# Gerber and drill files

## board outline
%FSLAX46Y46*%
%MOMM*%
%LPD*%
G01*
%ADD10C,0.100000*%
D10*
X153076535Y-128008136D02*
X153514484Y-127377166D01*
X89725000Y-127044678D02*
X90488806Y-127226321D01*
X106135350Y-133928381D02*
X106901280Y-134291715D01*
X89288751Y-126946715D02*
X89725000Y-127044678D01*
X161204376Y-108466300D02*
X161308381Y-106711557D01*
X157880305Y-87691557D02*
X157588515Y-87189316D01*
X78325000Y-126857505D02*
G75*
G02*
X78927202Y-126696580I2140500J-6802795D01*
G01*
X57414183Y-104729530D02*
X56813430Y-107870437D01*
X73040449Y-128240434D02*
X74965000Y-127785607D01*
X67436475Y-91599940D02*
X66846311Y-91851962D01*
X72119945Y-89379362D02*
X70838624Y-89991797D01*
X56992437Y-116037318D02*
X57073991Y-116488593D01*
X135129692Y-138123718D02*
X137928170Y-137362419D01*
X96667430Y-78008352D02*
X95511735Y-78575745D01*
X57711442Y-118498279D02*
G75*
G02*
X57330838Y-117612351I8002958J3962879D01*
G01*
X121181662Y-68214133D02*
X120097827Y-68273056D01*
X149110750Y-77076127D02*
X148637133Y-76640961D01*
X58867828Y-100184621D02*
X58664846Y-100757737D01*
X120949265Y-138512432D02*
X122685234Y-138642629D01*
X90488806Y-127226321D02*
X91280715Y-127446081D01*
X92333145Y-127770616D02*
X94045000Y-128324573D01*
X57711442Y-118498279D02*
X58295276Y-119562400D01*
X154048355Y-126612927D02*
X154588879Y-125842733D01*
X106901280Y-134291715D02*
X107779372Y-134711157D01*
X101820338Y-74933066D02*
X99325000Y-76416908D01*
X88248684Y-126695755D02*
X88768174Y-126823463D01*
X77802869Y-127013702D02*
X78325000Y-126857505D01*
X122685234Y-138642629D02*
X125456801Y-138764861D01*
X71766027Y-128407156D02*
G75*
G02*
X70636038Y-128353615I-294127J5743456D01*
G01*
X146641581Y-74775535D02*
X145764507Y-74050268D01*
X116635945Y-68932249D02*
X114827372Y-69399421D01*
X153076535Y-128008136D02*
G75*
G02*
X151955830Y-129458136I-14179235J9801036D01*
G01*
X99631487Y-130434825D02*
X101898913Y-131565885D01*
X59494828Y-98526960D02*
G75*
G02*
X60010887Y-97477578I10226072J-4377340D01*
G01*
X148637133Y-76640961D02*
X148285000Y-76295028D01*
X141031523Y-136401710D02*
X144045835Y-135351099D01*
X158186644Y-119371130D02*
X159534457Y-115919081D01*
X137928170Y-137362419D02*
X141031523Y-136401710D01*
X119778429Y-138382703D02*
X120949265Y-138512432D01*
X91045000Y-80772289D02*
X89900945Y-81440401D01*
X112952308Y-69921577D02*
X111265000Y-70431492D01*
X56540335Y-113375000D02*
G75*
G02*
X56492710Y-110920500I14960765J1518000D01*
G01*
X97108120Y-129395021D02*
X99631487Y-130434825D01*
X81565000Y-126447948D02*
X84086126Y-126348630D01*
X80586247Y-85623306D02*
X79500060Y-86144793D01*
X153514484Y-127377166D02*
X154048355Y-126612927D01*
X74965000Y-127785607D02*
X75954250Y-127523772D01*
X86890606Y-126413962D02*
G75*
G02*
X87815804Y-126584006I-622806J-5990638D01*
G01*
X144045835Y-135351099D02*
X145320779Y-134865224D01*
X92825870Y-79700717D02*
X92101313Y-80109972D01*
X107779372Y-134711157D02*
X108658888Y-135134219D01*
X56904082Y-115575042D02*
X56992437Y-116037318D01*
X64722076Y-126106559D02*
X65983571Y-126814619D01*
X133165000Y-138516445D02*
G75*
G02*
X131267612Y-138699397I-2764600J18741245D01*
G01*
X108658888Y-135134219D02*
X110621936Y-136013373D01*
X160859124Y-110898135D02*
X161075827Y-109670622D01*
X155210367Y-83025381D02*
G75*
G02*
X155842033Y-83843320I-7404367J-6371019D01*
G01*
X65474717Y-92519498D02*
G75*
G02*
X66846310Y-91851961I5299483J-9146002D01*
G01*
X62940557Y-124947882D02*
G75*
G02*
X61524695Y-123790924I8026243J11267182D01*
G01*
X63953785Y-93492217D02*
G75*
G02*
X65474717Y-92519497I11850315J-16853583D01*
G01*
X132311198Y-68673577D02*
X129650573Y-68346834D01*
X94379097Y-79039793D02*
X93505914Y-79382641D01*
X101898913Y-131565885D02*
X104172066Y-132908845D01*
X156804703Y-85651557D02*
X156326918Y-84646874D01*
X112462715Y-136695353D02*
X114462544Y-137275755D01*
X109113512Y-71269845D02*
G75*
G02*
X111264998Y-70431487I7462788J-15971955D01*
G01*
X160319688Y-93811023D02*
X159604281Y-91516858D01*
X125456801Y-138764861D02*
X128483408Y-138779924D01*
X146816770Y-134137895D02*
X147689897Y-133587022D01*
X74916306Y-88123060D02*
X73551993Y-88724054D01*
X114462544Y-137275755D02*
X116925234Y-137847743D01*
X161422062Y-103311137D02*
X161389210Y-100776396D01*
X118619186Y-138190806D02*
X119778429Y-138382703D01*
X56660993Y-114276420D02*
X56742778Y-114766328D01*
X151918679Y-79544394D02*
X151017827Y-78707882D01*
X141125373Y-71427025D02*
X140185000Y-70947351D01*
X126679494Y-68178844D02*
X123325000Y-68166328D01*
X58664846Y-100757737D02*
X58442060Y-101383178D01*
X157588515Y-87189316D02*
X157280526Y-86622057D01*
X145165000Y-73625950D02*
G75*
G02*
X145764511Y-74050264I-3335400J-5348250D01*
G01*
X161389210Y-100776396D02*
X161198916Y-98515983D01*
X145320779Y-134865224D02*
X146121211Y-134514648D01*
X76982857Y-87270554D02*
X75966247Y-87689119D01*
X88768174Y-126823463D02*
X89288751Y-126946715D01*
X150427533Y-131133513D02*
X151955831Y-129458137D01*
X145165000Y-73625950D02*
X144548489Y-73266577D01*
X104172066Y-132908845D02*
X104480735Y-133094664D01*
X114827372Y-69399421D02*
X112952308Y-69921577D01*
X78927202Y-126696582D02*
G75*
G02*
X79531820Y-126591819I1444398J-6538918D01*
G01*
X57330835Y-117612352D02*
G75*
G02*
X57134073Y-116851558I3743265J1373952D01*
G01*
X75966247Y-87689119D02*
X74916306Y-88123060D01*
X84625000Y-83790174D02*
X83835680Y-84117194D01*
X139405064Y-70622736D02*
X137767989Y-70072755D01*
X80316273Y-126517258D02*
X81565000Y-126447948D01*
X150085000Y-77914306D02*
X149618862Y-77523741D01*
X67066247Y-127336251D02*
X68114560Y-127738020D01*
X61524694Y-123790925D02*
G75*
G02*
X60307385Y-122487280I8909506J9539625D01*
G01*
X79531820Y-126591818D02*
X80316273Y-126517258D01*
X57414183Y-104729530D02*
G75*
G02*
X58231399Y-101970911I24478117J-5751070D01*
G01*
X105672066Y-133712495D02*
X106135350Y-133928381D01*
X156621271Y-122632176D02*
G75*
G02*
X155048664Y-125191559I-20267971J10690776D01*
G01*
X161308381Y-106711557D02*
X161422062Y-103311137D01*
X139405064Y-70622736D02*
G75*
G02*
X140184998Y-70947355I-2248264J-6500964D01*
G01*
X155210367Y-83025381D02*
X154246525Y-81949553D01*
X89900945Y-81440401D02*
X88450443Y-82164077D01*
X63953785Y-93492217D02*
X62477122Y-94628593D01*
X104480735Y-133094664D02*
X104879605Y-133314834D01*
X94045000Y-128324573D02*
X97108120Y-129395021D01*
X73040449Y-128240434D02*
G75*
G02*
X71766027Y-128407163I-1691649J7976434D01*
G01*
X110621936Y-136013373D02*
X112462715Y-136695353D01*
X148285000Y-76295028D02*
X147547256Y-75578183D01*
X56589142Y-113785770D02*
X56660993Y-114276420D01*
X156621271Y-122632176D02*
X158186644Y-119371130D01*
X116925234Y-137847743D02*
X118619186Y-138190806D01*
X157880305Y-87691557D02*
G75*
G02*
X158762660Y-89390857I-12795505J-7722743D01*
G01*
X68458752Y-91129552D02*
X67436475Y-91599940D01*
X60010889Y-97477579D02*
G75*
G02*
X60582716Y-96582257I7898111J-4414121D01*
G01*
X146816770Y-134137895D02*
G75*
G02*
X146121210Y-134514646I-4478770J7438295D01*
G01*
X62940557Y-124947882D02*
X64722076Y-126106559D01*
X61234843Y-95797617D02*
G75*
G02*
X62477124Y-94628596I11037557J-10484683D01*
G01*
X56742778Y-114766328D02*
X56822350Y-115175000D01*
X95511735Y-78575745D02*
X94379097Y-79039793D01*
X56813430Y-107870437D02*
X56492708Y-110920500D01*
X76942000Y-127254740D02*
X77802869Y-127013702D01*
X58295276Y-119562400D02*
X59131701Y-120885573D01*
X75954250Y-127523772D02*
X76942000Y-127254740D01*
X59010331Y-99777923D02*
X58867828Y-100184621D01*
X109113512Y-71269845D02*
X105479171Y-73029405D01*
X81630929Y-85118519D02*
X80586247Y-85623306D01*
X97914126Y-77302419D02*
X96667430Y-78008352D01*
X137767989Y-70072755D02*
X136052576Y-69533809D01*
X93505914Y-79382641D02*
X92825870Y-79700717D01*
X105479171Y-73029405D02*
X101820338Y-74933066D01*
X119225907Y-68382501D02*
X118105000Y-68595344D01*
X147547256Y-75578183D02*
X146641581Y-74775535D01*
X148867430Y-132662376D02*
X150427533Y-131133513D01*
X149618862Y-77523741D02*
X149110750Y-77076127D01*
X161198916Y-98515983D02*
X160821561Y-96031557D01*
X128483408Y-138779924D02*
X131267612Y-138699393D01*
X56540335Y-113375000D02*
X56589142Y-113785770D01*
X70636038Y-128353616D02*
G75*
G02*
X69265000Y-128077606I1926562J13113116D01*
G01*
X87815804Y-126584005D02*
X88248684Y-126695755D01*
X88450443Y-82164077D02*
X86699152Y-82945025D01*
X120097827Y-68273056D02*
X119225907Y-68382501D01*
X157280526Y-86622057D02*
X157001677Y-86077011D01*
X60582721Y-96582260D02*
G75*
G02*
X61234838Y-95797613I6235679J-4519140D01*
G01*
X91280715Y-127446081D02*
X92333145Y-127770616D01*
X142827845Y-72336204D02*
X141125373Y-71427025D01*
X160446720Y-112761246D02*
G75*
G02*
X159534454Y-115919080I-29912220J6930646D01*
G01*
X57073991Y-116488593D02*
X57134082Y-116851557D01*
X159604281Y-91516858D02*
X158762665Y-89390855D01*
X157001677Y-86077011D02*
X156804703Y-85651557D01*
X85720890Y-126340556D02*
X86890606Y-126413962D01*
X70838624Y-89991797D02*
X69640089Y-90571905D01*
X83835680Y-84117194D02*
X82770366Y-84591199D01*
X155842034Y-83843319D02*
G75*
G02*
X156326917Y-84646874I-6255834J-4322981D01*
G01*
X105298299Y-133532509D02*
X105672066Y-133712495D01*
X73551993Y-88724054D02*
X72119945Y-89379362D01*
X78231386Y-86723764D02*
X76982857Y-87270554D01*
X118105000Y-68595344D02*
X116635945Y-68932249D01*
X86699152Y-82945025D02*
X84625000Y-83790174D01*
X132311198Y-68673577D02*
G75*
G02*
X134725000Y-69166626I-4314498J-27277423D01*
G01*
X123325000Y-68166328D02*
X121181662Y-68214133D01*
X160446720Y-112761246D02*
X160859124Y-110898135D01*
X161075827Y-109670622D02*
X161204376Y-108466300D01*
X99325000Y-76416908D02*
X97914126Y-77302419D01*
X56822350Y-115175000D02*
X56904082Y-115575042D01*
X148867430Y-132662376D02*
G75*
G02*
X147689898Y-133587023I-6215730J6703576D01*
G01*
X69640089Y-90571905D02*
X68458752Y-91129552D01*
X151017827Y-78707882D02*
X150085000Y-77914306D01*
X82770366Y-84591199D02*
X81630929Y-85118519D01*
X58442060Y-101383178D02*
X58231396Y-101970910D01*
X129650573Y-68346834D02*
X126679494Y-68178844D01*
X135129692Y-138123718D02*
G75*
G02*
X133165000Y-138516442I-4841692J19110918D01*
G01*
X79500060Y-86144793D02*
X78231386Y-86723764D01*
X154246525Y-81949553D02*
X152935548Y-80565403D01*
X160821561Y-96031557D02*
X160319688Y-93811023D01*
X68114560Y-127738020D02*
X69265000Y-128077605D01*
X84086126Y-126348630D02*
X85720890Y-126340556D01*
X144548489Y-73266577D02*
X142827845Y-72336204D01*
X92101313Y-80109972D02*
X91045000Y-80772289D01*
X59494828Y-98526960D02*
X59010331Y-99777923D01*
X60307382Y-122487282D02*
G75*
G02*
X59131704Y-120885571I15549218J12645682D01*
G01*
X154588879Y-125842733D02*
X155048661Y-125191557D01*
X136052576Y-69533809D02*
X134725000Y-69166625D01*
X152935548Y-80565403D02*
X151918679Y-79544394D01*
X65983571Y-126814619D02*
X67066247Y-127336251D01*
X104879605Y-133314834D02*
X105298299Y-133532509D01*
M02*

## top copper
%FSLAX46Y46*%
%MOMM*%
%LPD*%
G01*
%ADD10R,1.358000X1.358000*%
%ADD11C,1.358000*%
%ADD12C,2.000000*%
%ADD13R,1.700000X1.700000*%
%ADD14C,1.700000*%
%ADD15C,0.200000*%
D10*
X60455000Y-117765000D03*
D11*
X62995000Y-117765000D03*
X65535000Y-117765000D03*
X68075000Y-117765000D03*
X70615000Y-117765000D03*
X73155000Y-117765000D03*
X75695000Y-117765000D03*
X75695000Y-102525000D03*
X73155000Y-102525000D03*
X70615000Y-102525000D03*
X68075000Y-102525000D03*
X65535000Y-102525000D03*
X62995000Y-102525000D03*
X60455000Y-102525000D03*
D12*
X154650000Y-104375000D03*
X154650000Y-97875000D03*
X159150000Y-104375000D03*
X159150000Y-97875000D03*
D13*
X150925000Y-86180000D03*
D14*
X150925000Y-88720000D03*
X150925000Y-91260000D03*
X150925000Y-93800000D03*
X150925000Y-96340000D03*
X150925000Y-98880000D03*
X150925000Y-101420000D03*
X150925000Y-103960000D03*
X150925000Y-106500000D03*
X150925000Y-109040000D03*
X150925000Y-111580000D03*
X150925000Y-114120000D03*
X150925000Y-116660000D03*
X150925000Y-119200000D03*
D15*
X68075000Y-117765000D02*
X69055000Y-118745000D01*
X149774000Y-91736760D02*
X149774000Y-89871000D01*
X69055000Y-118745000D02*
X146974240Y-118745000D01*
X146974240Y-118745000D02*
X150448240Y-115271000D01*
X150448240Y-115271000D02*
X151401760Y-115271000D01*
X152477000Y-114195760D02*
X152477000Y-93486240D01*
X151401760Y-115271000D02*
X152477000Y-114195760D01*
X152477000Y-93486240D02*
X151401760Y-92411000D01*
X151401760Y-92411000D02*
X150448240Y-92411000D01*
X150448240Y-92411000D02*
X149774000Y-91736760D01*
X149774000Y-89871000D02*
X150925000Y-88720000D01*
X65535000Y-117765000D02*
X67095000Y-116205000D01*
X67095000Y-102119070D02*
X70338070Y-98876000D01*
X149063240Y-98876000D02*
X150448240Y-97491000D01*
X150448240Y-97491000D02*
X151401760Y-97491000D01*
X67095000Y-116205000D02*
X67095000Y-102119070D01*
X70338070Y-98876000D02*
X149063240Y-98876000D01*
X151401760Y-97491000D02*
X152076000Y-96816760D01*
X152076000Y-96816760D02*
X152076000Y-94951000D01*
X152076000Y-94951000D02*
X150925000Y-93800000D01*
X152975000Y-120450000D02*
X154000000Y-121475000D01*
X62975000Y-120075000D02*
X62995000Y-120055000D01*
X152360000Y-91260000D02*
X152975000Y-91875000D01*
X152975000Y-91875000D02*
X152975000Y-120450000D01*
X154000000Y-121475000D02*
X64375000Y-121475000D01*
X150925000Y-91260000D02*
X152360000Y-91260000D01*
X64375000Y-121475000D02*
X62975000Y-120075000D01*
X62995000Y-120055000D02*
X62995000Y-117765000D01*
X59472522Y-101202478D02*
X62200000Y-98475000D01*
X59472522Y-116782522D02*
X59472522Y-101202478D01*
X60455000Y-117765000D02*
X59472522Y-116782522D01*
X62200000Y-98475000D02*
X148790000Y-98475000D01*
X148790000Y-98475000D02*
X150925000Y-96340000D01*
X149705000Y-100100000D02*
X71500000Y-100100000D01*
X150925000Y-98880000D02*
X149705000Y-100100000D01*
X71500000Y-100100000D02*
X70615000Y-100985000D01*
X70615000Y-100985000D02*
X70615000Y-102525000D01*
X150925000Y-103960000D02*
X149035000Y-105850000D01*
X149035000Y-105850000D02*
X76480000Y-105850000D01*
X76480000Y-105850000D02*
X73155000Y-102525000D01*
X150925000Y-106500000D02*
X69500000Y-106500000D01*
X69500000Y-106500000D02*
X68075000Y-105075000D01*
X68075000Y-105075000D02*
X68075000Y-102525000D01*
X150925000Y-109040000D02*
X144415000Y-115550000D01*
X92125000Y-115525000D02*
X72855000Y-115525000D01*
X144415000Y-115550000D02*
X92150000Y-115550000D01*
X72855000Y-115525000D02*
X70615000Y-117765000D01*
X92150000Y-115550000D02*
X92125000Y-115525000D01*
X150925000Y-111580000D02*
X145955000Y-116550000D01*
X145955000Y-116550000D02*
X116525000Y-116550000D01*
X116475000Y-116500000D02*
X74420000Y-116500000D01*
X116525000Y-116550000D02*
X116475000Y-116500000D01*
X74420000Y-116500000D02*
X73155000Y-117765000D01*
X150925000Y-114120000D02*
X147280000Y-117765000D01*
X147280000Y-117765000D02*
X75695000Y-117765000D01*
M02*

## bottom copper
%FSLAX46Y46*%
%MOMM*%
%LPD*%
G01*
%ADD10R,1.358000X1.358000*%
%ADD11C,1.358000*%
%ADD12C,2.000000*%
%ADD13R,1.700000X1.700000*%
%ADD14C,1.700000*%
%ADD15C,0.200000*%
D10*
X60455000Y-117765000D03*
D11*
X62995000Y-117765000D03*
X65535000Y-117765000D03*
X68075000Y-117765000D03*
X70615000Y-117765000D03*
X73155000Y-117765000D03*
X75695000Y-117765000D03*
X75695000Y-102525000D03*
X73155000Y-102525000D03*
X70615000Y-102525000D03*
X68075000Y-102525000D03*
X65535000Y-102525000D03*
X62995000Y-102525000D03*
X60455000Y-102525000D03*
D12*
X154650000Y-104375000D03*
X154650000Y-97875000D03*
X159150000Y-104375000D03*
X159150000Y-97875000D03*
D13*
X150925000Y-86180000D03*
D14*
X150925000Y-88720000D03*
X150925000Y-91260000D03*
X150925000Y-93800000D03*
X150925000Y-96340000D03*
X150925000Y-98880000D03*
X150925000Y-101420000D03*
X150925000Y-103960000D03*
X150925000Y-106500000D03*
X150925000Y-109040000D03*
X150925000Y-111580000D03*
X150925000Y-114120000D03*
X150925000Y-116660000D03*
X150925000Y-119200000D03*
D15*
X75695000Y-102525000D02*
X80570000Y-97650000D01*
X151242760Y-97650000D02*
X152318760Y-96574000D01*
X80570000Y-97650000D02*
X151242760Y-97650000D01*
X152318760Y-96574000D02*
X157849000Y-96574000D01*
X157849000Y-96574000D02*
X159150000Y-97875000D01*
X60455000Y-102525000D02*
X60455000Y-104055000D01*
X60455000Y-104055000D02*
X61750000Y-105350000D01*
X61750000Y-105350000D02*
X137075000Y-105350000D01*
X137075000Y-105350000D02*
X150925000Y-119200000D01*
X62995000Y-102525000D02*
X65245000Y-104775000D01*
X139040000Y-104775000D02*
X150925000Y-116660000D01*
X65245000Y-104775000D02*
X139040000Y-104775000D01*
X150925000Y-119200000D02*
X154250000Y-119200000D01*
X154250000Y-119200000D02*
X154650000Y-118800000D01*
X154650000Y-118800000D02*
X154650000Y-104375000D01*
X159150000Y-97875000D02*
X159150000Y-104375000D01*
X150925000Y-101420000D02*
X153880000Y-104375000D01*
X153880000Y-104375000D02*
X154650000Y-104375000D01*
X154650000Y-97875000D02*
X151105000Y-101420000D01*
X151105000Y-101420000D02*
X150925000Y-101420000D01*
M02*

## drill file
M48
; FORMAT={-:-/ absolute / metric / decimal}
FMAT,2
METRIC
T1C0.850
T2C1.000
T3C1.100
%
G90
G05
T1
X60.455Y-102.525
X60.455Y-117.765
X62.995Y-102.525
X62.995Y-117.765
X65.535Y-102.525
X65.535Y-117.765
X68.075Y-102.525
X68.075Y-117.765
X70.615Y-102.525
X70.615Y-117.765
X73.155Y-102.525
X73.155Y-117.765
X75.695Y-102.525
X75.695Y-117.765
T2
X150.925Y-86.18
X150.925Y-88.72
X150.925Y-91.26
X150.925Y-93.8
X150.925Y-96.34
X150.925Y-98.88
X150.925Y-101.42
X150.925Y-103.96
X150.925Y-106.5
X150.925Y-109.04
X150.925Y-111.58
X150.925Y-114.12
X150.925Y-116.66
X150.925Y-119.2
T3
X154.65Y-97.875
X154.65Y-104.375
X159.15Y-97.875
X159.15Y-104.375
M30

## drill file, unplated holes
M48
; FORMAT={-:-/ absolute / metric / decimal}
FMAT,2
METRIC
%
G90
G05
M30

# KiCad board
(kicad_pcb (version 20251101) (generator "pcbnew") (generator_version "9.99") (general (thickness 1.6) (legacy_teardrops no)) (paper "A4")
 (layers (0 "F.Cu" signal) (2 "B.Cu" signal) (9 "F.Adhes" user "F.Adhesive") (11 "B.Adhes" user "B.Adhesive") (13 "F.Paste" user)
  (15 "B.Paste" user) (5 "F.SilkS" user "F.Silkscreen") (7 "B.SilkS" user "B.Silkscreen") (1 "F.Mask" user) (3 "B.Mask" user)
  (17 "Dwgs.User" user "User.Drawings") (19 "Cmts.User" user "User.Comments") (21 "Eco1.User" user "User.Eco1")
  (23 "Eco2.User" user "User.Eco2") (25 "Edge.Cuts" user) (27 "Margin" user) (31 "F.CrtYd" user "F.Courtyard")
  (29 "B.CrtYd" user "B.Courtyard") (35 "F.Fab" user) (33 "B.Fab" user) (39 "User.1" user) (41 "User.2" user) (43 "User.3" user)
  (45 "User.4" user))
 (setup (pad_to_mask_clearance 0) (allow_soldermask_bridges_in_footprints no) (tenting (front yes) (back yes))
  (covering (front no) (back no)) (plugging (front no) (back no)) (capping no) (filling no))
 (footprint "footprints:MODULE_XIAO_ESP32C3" (layer "F.Cu") (at 68.0115 110.145 90)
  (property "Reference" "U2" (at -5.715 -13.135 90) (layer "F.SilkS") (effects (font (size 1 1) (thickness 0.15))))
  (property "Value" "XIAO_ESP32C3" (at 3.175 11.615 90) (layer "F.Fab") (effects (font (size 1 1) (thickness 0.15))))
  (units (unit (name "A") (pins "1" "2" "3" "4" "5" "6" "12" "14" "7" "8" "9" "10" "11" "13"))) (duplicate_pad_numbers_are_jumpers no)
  (pad "1" thru_hole rect (at -7.62 -7.5565 90) (size 1.358 1.358) (drill 0.85) (layers "*.Cu" "*.Mask") (remove_unused_layers no)
   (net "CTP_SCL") (solder_mask_margin 0.102) (tenting (front none) (back none)))
  (pad "2" thru_hole circle (at -7.62 -5.0165 90) (size 1.358 1.358) (drill 0.85) (layers "*.Cu" "*.Mask") (remove_unused_layers no)
   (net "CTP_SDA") (solder_mask_margin 0.102) (tenting (front none) (back none)))
  (pad "3" thru_hole circle (at -7.62 -2.4765 90) (size 1.358 1.358) (drill 0.85) (layers "*.Cu" "*.Mask") (remove_unused_layers no)
   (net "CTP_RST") (solder_mask_margin 0.102) (tenting (front none) (back none)))
  (pad "4" thru_hole circle (at -7.62 0.0635 90) (size 1.358 1.358) (drill 0.85) (layers "*.Cu" "*.Mask") (remove_unused_layers no)
   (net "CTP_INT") (solder_mask_margin 0.102) (tenting (front none) (back none)))
  (pad "5" thru_hole circle (at -7.62 2.6035 90) (size 1.358 1.358) (drill 0.85) (layers "*.Cu" "*.Mask") (remove_unused_layers no)
   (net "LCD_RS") (solder_mask_margin 0.102) (tenting (front none) (back none)))
  (pad "6" thru_hole circle (at -7.62 5.1435 90) (size 1.358 1.358) (drill 0.85) (layers "*.Cu" "*.Mask") (remove_unused_layers no)
   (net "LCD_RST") (solder_mask_margin 0.102) (tenting (front none) (back none)))
  (pad "7" thru_hole circle (at -7.62 7.6835 90) (size 1.358 1.358) (drill 0.85) (layers "*.Cu" "*.Mask") (remove_unused_layers no)
   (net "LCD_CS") (solder_mask_margin 0.102) (tenting (front none) (back none)))
  (pad "8" thru_hole circle (at 7.62 7.6835 90) (size 1.358 1.358) (drill 0.85) (layers "*.Cu" "*.Mask") (remove_unused_layers no)
   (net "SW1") (solder_mask_margin 0.102) (tenting (front none) (back none)))
  (pad "9" thru_hole circle (at 7.62 5.1435 90) (size 1.358 1.358) (drill 0.85) (layers "*.Cu" "*.Mask") (remove_unused_layers no)
   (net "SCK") (solder_mask_margin 0.102) (tenting (front none) (back none)))
  (pad "10" thru_hole circle (at 7.62 2.6035 90) (size 1.358 1.358) (drill 0.85) (layers "*.Cu" "*.Mask") (remove_unused_layers no)
   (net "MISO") (solder_mask_margin 0.102) (tenting (front none) (back none)))
  (pad "11" thru_hole circle (at 7.62 0.0635 90) (size 1.358 1.358) (drill 0.85) (layers "*.Cu" "*.Mask") (remove_unused_layers no)
   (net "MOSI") (solder_mask_margin 0.102) (tenting (front none) (back none)))
  (pad "12" thru_hole circle (at 7.62 -2.4765 90) (size 1.358 1.358) (drill 0.85) (layers "*.Cu" "*.Mask") (remove_unused_layers no)
   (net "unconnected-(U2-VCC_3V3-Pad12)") (solder_mask_margin 0.102) (tenting (front none) (back none)))
  (pad "13" thru_hole circle (at 7.62 -5.0165 90) (size 1.358 1.358) (drill 0.85) (layers "*.Cu" "*.Mask") (remove_unused_layers no)
   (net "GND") (solder_mask_margin 0.102) (tenting (front none) (back none)))
  (pad "14" thru_hole circle (at 7.62 -7.5565 90) (size 1.358 1.358) (drill 0.85) (layers "*.Cu" "*.Mask") (remove_unused_layers no)
   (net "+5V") (solder_mask_margin 0.102) (tenting (front none) (back none))))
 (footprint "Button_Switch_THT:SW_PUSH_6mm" (layer "F.Cu") (at 154.65 104.375 90)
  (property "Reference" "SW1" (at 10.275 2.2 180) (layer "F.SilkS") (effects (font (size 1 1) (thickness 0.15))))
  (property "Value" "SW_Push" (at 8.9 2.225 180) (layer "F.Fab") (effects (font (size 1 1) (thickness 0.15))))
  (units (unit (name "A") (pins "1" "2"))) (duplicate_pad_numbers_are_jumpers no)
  (pad "1" thru_hole circle (at 0 0 180) (size 2 2) (drill 1.1) (layers "*.Cu" "*.Mask") (remove_unused_layers no) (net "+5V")
   (tenting (front none) (back none)))
  (pad "1" thru_hole circle (at 6.5 0 180) (size 2 2) (drill 1.1) (layers "*.Cu" "*.Mask") (remove_unused_layers no) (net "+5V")
   (tenting (front none) (back none)))
  (pad "2" thru_hole circle (at 0 4.5 180) (size 2 2) (drill 1.1) (layers "*.Cu" "*.Mask") (remove_unused_layers no) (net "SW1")
   (tenting (front none) (back none)))
  (pad "2" thru_hole circle (at 6.5 4.5 180) (size 2 2) (drill 1.1) (layers "*.Cu" "*.Mask") (remove_unused_layers no) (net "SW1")
   (tenting (front none) (back none))))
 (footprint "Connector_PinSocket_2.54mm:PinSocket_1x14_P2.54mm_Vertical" (layer "F.Cu") (at 150.925 86.18)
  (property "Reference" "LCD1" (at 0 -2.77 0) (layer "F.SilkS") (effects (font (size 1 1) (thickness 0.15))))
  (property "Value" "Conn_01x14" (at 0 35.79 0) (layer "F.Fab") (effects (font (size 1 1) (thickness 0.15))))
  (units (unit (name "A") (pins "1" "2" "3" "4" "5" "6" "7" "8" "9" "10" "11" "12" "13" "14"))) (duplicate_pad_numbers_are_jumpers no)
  (pad "1" thru_hole rect (at 0 0) (size 1.7 1.7) (drill 1) (layers "*.Cu" "*.Mask") (remove_unused_layers no)
   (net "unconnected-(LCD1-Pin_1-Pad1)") (tenting (front none) (back none)))
  (pad "2" thru_hole circle (at 0 2.54) (size 1.7 1.7) (drill 1) (layers "*.Cu" "*.Mask") (remove_unused_layers no) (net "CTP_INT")
   (tenting (front none) (back none)))
  (pad "3" thru_hole circle (at 0 5.08) (size 1.7 1.7) (drill 1) (layers "*.Cu" "*.Mask") (remove_unused_layers no) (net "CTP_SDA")
   (tenting (front none) (back none)))
  (pad "4" thru_hole circle (at 0 7.62) (size 1.7 1.7) (drill 1) (layers "*.Cu" "*.Mask") (remove_unused_layers no) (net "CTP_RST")
   (tenting (front none) (back none)))
  (pad "5" thru_hole circle (at 0 10.16) (size 1.7 1.7) (drill 1) (layers "*.Cu" "*.Mask") (remove_unused_layers no) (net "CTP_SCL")
   (tenting (front none) (back none)))
  (pad "6" thru_hole circle (at 0 12.7) (size 1.7 1.7) (drill 1) (layers "*.Cu" "*.Mask") (remove_unused_layers no) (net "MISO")
   (tenting (front none) (back none)))
  (pad "7" thru_hole circle (at 0 15.24) (size 1.7 1.7) (drill 1) (layers "*.Cu" "*.Mask") (remove_unused_layers no) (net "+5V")
   (tenting (front none) (back none)))
  (pad "8" thru_hole circle (at 0 17.78) (size 1.7 1.7) (drill 1) (layers "*.Cu" "*.Mask") (remove_unused_layers no) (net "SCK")
   (tenting (front none) (back none)))
  (pad "9" thru_hole circle (at 0 20.32) (size 1.7 1.7) (drill 1) (layers "*.Cu" "*.Mask") (remove_unused_layers no) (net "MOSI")
   (tenting (front none) (back none)))
  (pad "10" thru_hole circle (at 0 22.86) (size 1.7 1.7) (drill 1) (layers "*.Cu" "*.Mask") (remove_unused_layers no) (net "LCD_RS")
   (tenting (front none) (back none)))
  (pad "11" thru_hole circle (at 0 25.4) (size 1.7 1.7) (drill 1) (layers "*.Cu" "*.Mask") (remove_unused_layers no) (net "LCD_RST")
   (tenting (front none) (back none)))
  (pad "12" thru_hole circle (at 0 27.94) (size 1.7 1.7) (drill 1) (layers "*.Cu" "*.Mask") (remove_unused_layers no) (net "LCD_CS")
   (tenting (front none) (back none)))
  (pad "13" thru_hole circle (at 0 30.48) (size 1.7 1.7) (drill 1) (layers "*.Cu" "*.Mask") (remove_unused_layers no) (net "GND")
   (tenting (front none) (back none)))
  (pad "14" thru_hole circle (at 0 33.02) (size 1.7 1.7) (drill 1) (layers "*.Cu" "*.Mask") (remove_unused_layers no) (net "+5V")
   (tenting (front none) (back none))))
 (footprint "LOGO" (layer "B.Cu") (at 118.27759 103.45 -90)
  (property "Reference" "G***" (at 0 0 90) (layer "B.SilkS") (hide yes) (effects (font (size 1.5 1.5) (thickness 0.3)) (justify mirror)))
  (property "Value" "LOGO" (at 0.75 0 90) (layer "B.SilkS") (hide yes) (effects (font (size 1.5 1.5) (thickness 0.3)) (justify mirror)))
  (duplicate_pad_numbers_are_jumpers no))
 (gr_line (start 153.076535 128.008136) (end 153.514484 127.377166) (stroke (width 0.1) (type default)) (layer "Edge.Cuts"))
 (gr_line (start 89.725 127.044678) (end 90.488806 127.226321) (stroke (width 0.1) (type default)) (layer "Edge.Cuts"))
 (gr_line (start 106.13535 133.928381) (end 106.90128 134.291715) (stroke (width 0.1) (type default)) (layer "Edge.Cuts"))
 (gr_line (start 89.288751 126.946715) (end 89.725 127.044678) (stroke (width 0.1) (type default)) (layer "Edge.Cuts"))
 (gr_line (start 161.204376 108.4663) (end 161.308381 106.711557) (stroke (width 0.1) (type default)) (layer "Edge.Cuts"))
 (gr_line (start 157.880305 87.691557) (end 157.588515 87.189316) (stroke (width 0.1) (type default)) (layer "Edge.Cuts"))
 (gr_arc (start 78.325 126.857505) (mid 78.624342 126.770461) (end 78.927202 126.696582) (stroke (width 0.1) (type default))
  (layer "Edge.Cuts"))
 (gr_line (start 57.414183 104.72953) (end 56.81343 107.870437) (stroke (width 0.1) (type default)) (layer "Edge.Cuts"))
 (gr_line (start 73.040449 128.240434) (end 74.965 127.785607) (stroke (width 0.1) (type default)) (layer "Edge.Cuts"))
 (gr_line (start 67.436475 91.59994) (end 66.846311 91.851962) (stroke (width 0.1) (type default)) (layer "Edge.Cuts"))
 (gr_line (start 72.119945 89.379362) (end 70.838624 89.991797) (stroke (width 0.1) (type default)) (layer "Edge.Cuts"))
 (gr_line (start 56.992437 116.037318) (end 57.073991 116.488593) (stroke (width 0.1) (type default)) (layer "Edge.Cuts"))
 (gr_line (start 135.129692 138.123718) (end 137.92817 137.362419) (stroke (width 0.1) (type default)) (layer "Edge.Cuts"))
 (gr_line (start 96.66743 78.008352) (end 95.511735 78.575745) (stroke (width 0.1) (type default)) (layer "Edge.Cuts"))
 (gr_arc (start 57.711442 118.498279) (mid 57.509173 118.060456) (end 57.330835 117.612352) (stroke (width 0.1) (type default))
  (layer "Edge.Cuts"))
 (gr_line (start 121.181662 68.214133) (end 120.097827 68.273056) (stroke (width 0.1) (type default)) (layer "Edge.Cuts"))
 (gr_line (start 149.11075 77.076127) (end 148.637133 76.640961) (stroke (width 0.1) (type default)) (layer "Edge.Cuts"))
 (gr_line (start 58.867828 100.184621) (end 58.664846 100.757737) (stroke (width 0.1) (type default)) (layer "Edge.Cuts"))
 (gr_line (start 120.949265 138.512432) (end 122.685234 138.642629) (stroke (width 0.1) (type default)) (layer "Edge.Cuts"))
 (gr_line (start 90.488806 127.226321) (end 91.280715 127.446081) (stroke (width 0.1) (type default)) (layer "Edge.Cuts"))
 (gr_line (start 92.333145 127.770616) (end 94.045 128.324573) (stroke (width 0.1) (type default)) (layer "Edge.Cuts"))
 (gr_line (start 57.711442 118.498279) (end 58.295276 119.5624) (stroke (width 0.1) (type default)) (layer "Edge.Cuts"))
 (gr_line (start 154.048355 126.612927) (end 154.588879 125.842733) (stroke (width 0.1) (type default)) (layer "Edge.Cuts"))
 (gr_line (start 106.90128 134.291715) (end 107.779372 134.711157) (stroke (width 0.1) (type default)) (layer "Edge.Cuts"))
 (gr_line (start 101.820338 74.933066) (end 99.325 76.416908) (stroke (width 0.1) (type default)) (layer "Edge.Cuts"))
 (gr_line (start 88.248684 126.695755) (end 88.768174 126.823463) (stroke (width 0.1) (type default)) (layer "Edge.Cuts"))
 (gr_line (start 77.802869 127.013702) (end 78.325 126.857505) (stroke (width 0.1) (type default)) (layer "Edge.Cuts"))
 (gr_line (start 122.685234 138.642629) (end 125.456801 138.764861) (stroke (width 0.1) (type default)) (layer "Edge.Cuts"))
 (gr_arc (start 71.766027 128.407156) (mid 71.199713 128.408238) (end 70.636038 128.353616) (stroke (width 0.1) (type default))
  (layer "Edge.Cuts"))
 (gr_line (start 146.641581 74.775535) (end 145.764507 74.050268) (stroke (width 0.1) (type default)) (layer "Edge.Cuts"))
 (gr_line (start 116.635945 68.932249) (end 114.827372 69.399421) (stroke (width 0.1) (type default)) (layer "Edge.Cuts"))
 (gr_arc (start 153.076535 128.008136) (mid 152.535467 128.748041) (end 151.955831 129.458137) (stroke (width 0.1) (type default))
  (layer "Edge.Cuts"))
 (gr_line (start 99.631487 130.434825) (end 101.898913 131.565885) (stroke (width 0.1) (type default)) (layer "Edge.Cuts"))
 (gr_arc (start 59.494828 98.52696) (mid 59.739059 97.995483) (end 60.010889 97.477579) (stroke (width 0.1) (type default))
  (layer "Edge.Cuts"))
 (gr_line (start 148.637133 76.640961) (end 148.285 76.295028) (stroke (width 0.1) (type default)) (layer "Edge.Cuts"))
 (gr_line (start 141.031523 136.40171) (end 144.045835 135.351099) (stroke (width 0.1) (type default)) (layer "Edge.Cuts"))
 (gr_line (start 158.186644 119.37113) (end 159.534457 115.919081) (stroke (width 0.1) (type default)) (layer "Edge.Cuts"))
 (gr_line (start 137.92817 137.362419) (end 141.031523 136.40171) (stroke (width 0.1) (type default)) (layer "Edge.Cuts"))
 (gr_line (start 119.778429 138.382703) (end 120.949265 138.512432) (stroke (width 0.1) (type default)) (layer "Edge.Cuts"))
 (gr_line (start 91.045 80.772289) (end 89.900945 81.440401) (stroke (width 0.1) (type default)) (layer "Edge.Cuts"))
 (gr_line (start 112.952308 69.921577) (end 111.265 70.431492) (stroke (width 0.1) (type default)) (layer "Edge.Cuts"))
 (gr_arc (start 56.540335 113.375) (mid 56.466349 112.148724) (end 56.492708 110.9205) (stroke (width 0.1) (type default))
  (layer "Edge.Cuts"))
 (gr_line (start 97.10812 129.395021) (end 99.631487 130.434825) (stroke (width 0.1) (type default)) (layer "Edge.Cuts"))
 (gr_line (start 81.565 126.447948) (end 84.086126 126.34863) (stroke (width 0.1) (type default)) (layer "Edge.Cuts"))
 (gr_line (start 80.586247 85.623306) (end 79.50006 86.144793) (stroke (width 0.1) (type default)) (layer "Edge.Cuts"))
 (gr_line (start 153.514484 127.377166) (end 154.048355 126.612927) (stroke (width 0.1) (type default)) (layer "Edge.Cuts"))
 (gr_line (start 74.965 127.785607) (end 75.95425 127.523772) (stroke (width 0.1) (type default)) (layer "Edge.Cuts"))
 (gr_arc (start 86.890606 126.413962) (mid 87.35653 126.480893) (end 87.815804 126.584005) (stroke (width 0.1) (type default))
  (layer "Edge.Cuts"))
 (gr_line (start 144.045835 135.351099) (end 145.320779 134.865224) (stroke (width 0.1) (type default)) (layer "Edge.Cuts"))
 (gr_line (start 92.82587 79.700717) (end 92.101313 80.109972) (stroke (width 0.1) (type default)) (layer "Edge.Cuts"))
 (gr_line (start 107.779372 134.711157) (end 108.658888 135.134219) (stroke (width 0.1) (type default)) (layer "Edge.Cuts"))
 (gr_line (start 56.904082 115.575042) (end 56.992437 116.037318) (stroke (width 0.1) (type default)) (layer "Edge.Cuts"))
 (gr_line (start 64.722076 126.106559) (end 65.983571 126.814619) (stroke (width 0.1) (type default)) (layer "Edge.Cuts"))
 (gr_arc (start 133.165 138.516445) (mid 132.218609 138.631799) (end 131.267612 138.699393) (stroke (width 0.1) (type default))
  (layer "Edge.Cuts"))
 (gr_line (start 108.658888 135.134219) (end 110.621936 136.013373) (stroke (width 0.1) (type default)) (layer "Edge.Cuts"))
 (gr_line (start 160.859124 110.898135) (end 161.075827 109.670622) (stroke (width 0.1) (type default)) (layer "Edge.Cuts"))
 (gr_arc (start 155.210367 83.025381) (mid 155.537025 83.42599) (end 155.842034 83.843319) (stroke (width 0.1) (type default))
  (layer "Edge.Cuts"))
 (gr_arc (start 65.474717 92.519498) (mid 66.148457 92.160956) (end 66.846311 91.851962) (stroke (width 0.1) (type default))
  (layer "Edge.Cuts"))
 (gr_arc (start 62.940557 124.947882) (mid 62.21349 124.392822) (end 61.524694 123.790925) (stroke (width 0.1) (type default))
  (layer "Edge.Cuts"))
 (gr_arc (start 63.953785 93.492217) (mid 64.703591 92.98919) (end 65.474717 92.519498) (stroke (width 0.1) (type default))
  (layer "Edge.Cuts"))
 (gr_line (start 132.311198 68.673577) (end 129.650573 68.346834) (stroke (width 0.1) (type default)) (layer "Edge.Cuts"))
 (gr_line (start 94.379097 79.039793) (end 93.505914 79.382641) (stroke (width 0.1) (type default)) (layer "Edge.Cuts"))
 (gr_line (start 101.898913 131.565885) (end 104.172066 132.908845) (stroke (width 0.1) (type default)) (layer "Edge.Cuts"))
 (gr_line (start 156.804703 85.651557) (end 156.326918 84.646874) (stroke (width 0.1) (type default)) (layer "Edge.Cuts"))
 (gr_line (start 112.462715 136.695353) (end 114.462544 137.275755) (stroke (width 0.1) (type default)) (layer "Edge.Cuts"))
 (gr_arc (start 109.113512 71.269845) (mid 110.175516 70.815406) (end 111.265 70.431492) (stroke (width 0.1) (type default))
  (layer "Edge.Cuts"))
 (gr_line (start 160.319688 93.811023) (end 159.604281 91.516858) (stroke (width 0.1) (type default)) (layer "Edge.Cuts"))
 (gr_line (start 125.456801 138.764861) (end 128.483408 138.779924) (stroke (width 0.1) (type default)) (layer "Edge.Cuts"))
 (gr_line (start 146.81677 134.137895) (end 147.689897 133.587022) (stroke (width 0.1) (type default)) (layer "Edge.Cuts"))
 (gr_line (start 74.916306 88.12306) (end 73.551993 88.724054) (stroke (width 0.1) (type default)) (layer "Edge.Cuts"))
 (gr_line (start 114.462544 137.275755) (end 116.925234 137.847743) (stroke (width 0.1) (type default)) (layer "Edge.Cuts"))
 (gr_line (start 161.422062 103.311137) (end 161.38921 100.776396) (stroke (width 0.1) (type default)) (layer "Edge.Cuts"))
 (gr_line (start 118.619186 138.190806) (end 119.778429 138.382703) (stroke (width 0.1) (type default)) (layer "Edge.Cuts"))
 (gr_line (start 56.660993 114.27642) (end 56.742778 114.766328) (stroke (width 0.1) (type default)) (layer "Edge.Cuts"))
 (gr_line (start 151.918679 79.544394) (end 151.017827 78.707882) (stroke (width 0.1) (type default)) (layer "Edge.Cuts"))
 (gr_line (start 141.125373 71.427025) (end 140.185 70.947351) (stroke (width 0.1) (type default)) (layer "Edge.Cuts"))
 (gr_line (start 126.679494 68.178844) (end 123.325 68.166328) (stroke (width 0.1) (type default)) (layer "Edge.Cuts"))
 (gr_line (start 58.664846 100.757737) (end 58.44206 101.383178) (stroke (width 0.1) (type default)) (layer "Edge.Cuts"))
 (gr_line (start 157.588515 87.189316) (end 157.280526 86.622057) (stroke (width 0.1) (type default)) (layer "Edge.Cuts"))
 (gr_arc (start 145.165 73.62595) (mid 145.470939 73.829369) (end 145.764507 74.050268) (stroke (width 0.1) (type default))
  (layer "Edge.Cuts"))
 (gr_line (start 161.38921 100.776396) (end 161.198916 98.515983) (stroke (width 0.1) (type default)) (layer "Edge.Cuts"))
 (gr_line (start 145.320779 134.865224) (end 146.121211 134.514648) (stroke (width 0.1) (type default)) (layer "Edge.Cuts"))
 (gr_line (start 76.982857 87.270554) (end 75.966247 87.689119) (stroke (width 0.1) (type default)) (layer "Edge.Cuts"))
 (gr_line (start 88.768174 126.823463) (end 89.288751 126.946715) (stroke (width 0.1) (type default)) (layer "Edge.Cuts"))
 (gr_line (start 150.427533 131.133513) (end 151.955831 129.458137) (stroke (width 0.1) (type default)) (layer "Edge.Cuts"))
 (gr_line (start 145.165 73.62595) (end 144.548489 73.266577) (stroke (width 0.1) (type default)) (layer "Edge.Cuts"))
 (gr_line (start 104.172066 132.908845) (end 104.480735 133.094664) (stroke (width 0.1) (type default)) (layer "Edge.Cuts"))
 (gr_line (start 114.827372 69.399421) (end 112.952308 69.921577) (stroke (width 0.1) (type default)) (layer "Edge.Cuts"))
 (gr_arc (start 78.927202 126.696582) (mid 79.22831 126.637271) (end 79.53182 126.591818) (stroke (width 0.1) (type default))
  (layer "Edge.Cuts"))
 (gr_arc (start 57.330835 117.612352) (mid 57.213671 117.236813) (end 57.134082 116.851557) (stroke (width 0.1) (type default))
  (layer "Edge.Cuts"))
 (gr_line (start 75.966247 87.689119) (end 74.916306 88.12306) (stroke (width 0.1) (type default)) (layer "Edge.Cuts"))
 (gr_line (start 84.625 83.790174) (end 83.83568 84.117194) (stroke (width 0.1) (type default)) (layer "Edge.Cuts"))
 (gr_line (start 139.405064 70.622736) (end 137.767989 70.072755) (stroke (width 0.1) (type default)) (layer "Edge.Cuts"))
 (gr_line (start 80.316273 126.517258) (end 81.565 126.447948) (stroke (width 0.1) (type default)) (layer "Edge.Cuts"))
 (gr_line (start 150.085 77.914306) (end 149.618862 77.523741) (stroke (width 0.1) (type default)) (layer "Edge.Cuts"))
 (gr_line (start 67.066247 127.336251) (end 68.11456 127.73802) (stroke (width 0.1) (type default)) (layer "Edge.Cuts"))
 (gr_arc (start 61.524694 123.790925) (mid 60.893745 123.15992) (end 60.307382 122.487282) (stroke (width 0.1) (type default))
  (layer "Edge.Cuts"))
 (gr_line (start 79.53182 126.591818) (end 80.316273 126.517258) (stroke (width 0.1) (type default)) (layer "Edge.Cuts"))
 (gr_arc (start 57.414183 104.72953) (mid 57.783301 103.338522) (end 58.231396 101.97091) (stroke (width 0.1) (type default))
  (layer "Edge.Cuts"))
 (gr_line (start 105.672066 133.712495) (end 106.13535 133.928381) (stroke (width 0.1) (type default)) (layer "Edge.Cuts"))
 (gr_arc (start 156.621271 122.632176) (mid 155.87695 123.937664) (end 155.048661 125.191557) (stroke (width 0.1) (type default))
  (layer "Edge.Cuts"))
 (gr_line (start 161.308381 106.711557) (end 161.422062 103.311137) (stroke (width 0.1) (type default)) (layer "Edge.Cuts"))
 (gr_arc (start 139.405064 70.622736) (mid 139.80002 70.773059) (end 140.185 70.947351) (stroke (width 0.1) (type default))
  (layer "Edge.Cuts"))
 (gr_line (start 155.210367 83.025381) (end 154.246525 81.949553) (stroke (width 0.1) (type default)) (layer "Edge.Cuts"))
 (gr_line (start 89.900945 81.440401) (end 88.450443 82.164077) (stroke (width 0.1) (type default)) (layer "Edge.Cuts"))
 (gr_line (start 63.953785 93.492217) (end 62.477122 94.628593) (stroke (width 0.1) (type default)) (layer "Edge.Cuts"))
 (gr_line (start 104.480735 133.094664) (end 104.879605 133.314834) (stroke (width 0.1) (type default)) (layer "Edge.Cuts"))
 (gr_line (start 94.045 128.324573) (end 97.10812 129.395021) (stroke (width 0.1) (type default)) (layer "Edge.Cuts"))
 (gr_arc (start 73.040449 128.240434) (mid 72.406528 128.348945) (end 71.766027 128.407156) (stroke (width 0.1) (type default))
  (layer "Edge.Cuts"))
 (gr_line (start 110.621936 136.013373) (end 112.462715 136.695353) (stroke (width 0.1) (type default)) (layer "Edge.Cuts"))
 (gr_line (start 148.285 76.295028) (end 147.547256 75.578183) (stroke (width 0.1) (type default)) (layer "Edge.Cuts"))
 (gr_line (start 56.589142 113.78577) (end 56.660993 114.27642) (stroke (width 0.1) (type default)) (layer "Edge.Cuts"))
 (gr_line (start 156.621271 122.632176) (end 158.186644 119.37113) (stroke (width 0.1) (type default)) (layer "Edge.Cuts"))
 (gr_line (start 116.925234 137.847743) (end 118.619186 138.190806) (stroke (width 0.1) (type default)) (layer "Edge.Cuts"))
 (gr_arc (start 157.880305 87.691557) (mid 158.348726 88.527061) (end 158.762665 89.390855) (stroke (width 0.1) (type default))
  (layer "Edge.Cuts"))
 (gr_line (start 68.458752 91.129552) (end 67.436475 91.59994) (stroke (width 0.1) (type default)) (layer "Edge.Cuts"))
 (gr_arc (start 60.010889 97.477579) (mid 60.283653 97.02152) (end 60.582721 96.58226) (stroke (width 0.1) (type default))
  (layer "Edge.Cuts"))
 (gr_arc (start 146.81677 134.137895) (mid 146.473283 134.334197) (end 146.121211 134.514648) (stroke (width 0.1) (type default))
  (layer "Edge.Cuts"))
 (gr_line (start 62.940557 124.947882) (end 64.722076 126.106559) (stroke (width 0.1) (type default)) (layer "Edge.Cuts"))
 (gr_arc (start 61.234843 95.797617) (mid 61.839596 95.195691) (end 62.477122 94.628593) (stroke (width 0.1) (type default))
  (layer "Edge.Cuts"))
 (gr_line (start 56.742778 114.766328) (end 56.82235 115.175) (stroke (width 0.1) (type default)) (layer "Edge.Cuts"))
 (gr_line (start 95.511735 78.575745) (end 94.379097 79.039793) (stroke (width 0.1) (type default)) (layer "Edge.Cuts"))
 (gr_line (start 56.81343 107.870437) (end 56.492708 110.9205) (stroke (width 0.1) (type default)) (layer "Edge.Cuts"))
 (gr_line (start 76.942 127.25474) (end 77.802869 127.013702) (stroke (width 0.1) (type default)) (layer "Edge.Cuts"))
 (gr_line (start 58.295276 119.5624) (end 59.131701 120.885573) (stroke (width 0.1) (type default)) (layer "Edge.Cuts"))
 (gr_line (start 75.95425 127.523772) (end 76.942 127.25474) (stroke (width 0.1) (type default)) (layer "Edge.Cuts"))
 (gr_line (start 59.010331 99.777923) (end 58.867828 100.184621) (stroke (width 0.1) (type default)) (layer "Edge.Cuts"))
 (gr_line (start 109.113512 71.269845) (end 105.479171 73.029405) (stroke (width 0.1) (type default)) (layer "Edge.Cuts"))
 (gr_line (start 81.630929 85.118519) (end 80.586247 85.623306) (stroke (width 0.1) (type default)) (layer "Edge.Cuts"))
 (gr_line (start 97.914126 77.302419) (end 96.66743 78.008352) (stroke (width 0.1) (type default)) (layer "Edge.Cuts"))
 (gr_line (start 137.767989 70.072755) (end 136.052576 69.533809) (stroke (width 0.1) (type default)) (layer "Edge.Cuts"))
 (gr_line (start 93.505914 79.382641) (end 92.82587 79.700717) (stroke (width 0.1) (type default)) (layer "Edge.Cuts"))
 (gr_line (start 105.479171 73.029405) (end 101.820338 74.933066) (stroke (width 0.1) (type default)) (layer "Edge.Cuts"))
 (gr_line (start 119.225907 68.382501) (end 118.105 68.595344) (stroke (width 0.1) (type default)) (layer "Edge.Cuts"))
 (gr_line (start 147.547256 75.578183) (end 146.641581 74.775535) (stroke (width 0.1) (type default)) (layer "Edge.Cuts"))
 (gr_line (start 148.86743 132.662376) (end 150.427533 131.133513) (stroke (width 0.1) (type default)) (layer "Edge.Cuts"))
 (gr_line (start 149.618862 77.523741) (end 149.11075 77.076127) (stroke (width 0.1) (type default)) (layer "Edge.Cuts"))
 (gr_line (start 161.198916 98.515983) (end 160.821561 96.031557) (stroke (width 0.1) (type default)) (layer "Edge.Cuts"))
 (gr_line (start 128.483408 138.779924) (end 131.267612 138.699393) (stroke (width 0.1) (type default)) (layer "Edge.Cuts"))
 (gr_line (start 56.540335 113.375) (end 56.589142 113.78577) (stroke (width 0.1) (type default)) (layer "Edge.Cuts"))
 (gr_arc (start 70.636038 128.353616) (mid 69.946876 128.233707) (end 69.265 128.077605) (stroke (width 0.1) (type default))
  (layer "Edge.Cuts"))
 (gr_line (start 87.815804 126.584005) (end 88.248684 126.695755) (stroke (width 0.1) (type default)) (layer "Edge.Cuts"))
 (gr_line (start 88.450443 82.164077) (end 86.699152 82.945025) (stroke (width 0.1) (type default)) (layer "Edge.Cuts"))
 (gr_line (start 120.097827 68.273056) (end 119.225907 68.382501) (stroke (width 0.1) (type default)) (layer "Edge.Cuts"))
 (gr_line (start 157.280526 86.622057) (end 157.001677 86.077011) (stroke (width 0.1) (type default)) (layer "Edge.Cuts"))
 (gr_arc (start 60.582721 96.58226) (mid 60.895774 96.179127) (end 61.234843 95.797617) (stroke (width 0.1) (type default))
  (layer "Edge.Cuts"))
 (gr_line (start 91.280715 127.446081) (end 92.333145 127.770616) (stroke (width 0.1) (type default)) (layer "Edge.Cuts"))
 (gr_line (start 142.827845 72.336204) (end 141.125373 71.427025) (stroke (width 0.1) (type default)) (layer "Edge.Cuts"))
 (gr_arc (start 160.44672 112.761246) (mid 160.032875 114.35238) (end 159.534457 115.919081) (stroke (width 0.1) (type default))
  (layer "Edge.Cuts"))
 (gr_line (start 57.073991 116.488593) (end 57.134082 116.851557) (stroke (width 0.1) (type default)) (layer "Edge.Cuts"))
 (gr_line (start 159.604281 91.516858) (end 158.762665 89.390855) (stroke (width 0.1) (type default)) (layer "Edge.Cuts"))
 (gr_line (start 157.001677 86.077011) (end 156.804703 85.651557) (stroke (width 0.1) (type default)) (layer "Edge.Cuts"))
 (gr_line (start 85.72089 126.340556) (end 86.890606 126.413962) (stroke (width 0.1) (type default)) (layer "Edge.Cuts"))
 (gr_line (start 70.838624 89.991797) (end 69.640089 90.571905) (stroke (width 0.1) (type default)) (layer "Edge.Cuts"))
 (gr_line (start 83.83568 84.117194) (end 82.770366 84.591199) (stroke (width 0.1) (type default)) (layer "Edge.Cuts"))
 (gr_arc (start 155.842034 83.843319) (mid 156.096885 84.237609) (end 156.326918 84.646874) (stroke (width 0.1) (type default))
  (layer "Edge.Cuts"))
 (gr_line (start 105.298299 133.532509) (end 105.672066 133.712495) (stroke (width 0.1) (type default)) (layer "Edge.Cuts"))
 (gr_line (start 73.551993 88.724054) (end 72.119945 89.379362) (stroke (width 0.1) (type default)) (layer "Edge.Cuts"))
 (gr_line (start 78.231386 86.723764) (end 76.982857 87.270554) (stroke (width 0.1) (type default)) (layer "Edge.Cuts"))
 (gr_line (start 118.105 68.595344) (end 116.635945 68.932249) (stroke (width 0.1) (type default)) (layer "Edge.Cuts"))
 (gr_line (start 86.699152 82.945025) (end 84.625 83.790174) (stroke (width 0.1) (type default)) (layer "Edge.Cuts"))
 (gr_arc (start 132.311198 68.673577) (mid 133.5236 68.893171) (end 134.725 69.166625) (stroke (width 0.1) (type default))
  (layer "Edge.Cuts"))
 (gr_line (start 123.325 68.166328) (end 121.181662 68.214133) (stroke (width 0.1) (type default)) (layer "Edge.Cuts"))
 (gr_line (start 160.44672 112.761246) (end 160.859124 110.898135) (stroke (width 0.1) (type default)) (layer "Edge.Cuts"))
 (gr_line (start 161.075827 109.670622) (end 161.204376 108.4663) (stroke (width 0.1) (type default)) (layer "Edge.Cuts"))
 (gr_line (start 99.325 76.416908) (end 97.914126 77.302419) (stroke (width 0.1) (type default)) (layer "Edge.Cuts"))
 (gr_line (start 56.82235 115.175) (end 56.904082 115.575042) (stroke (width 0.1) (type default)) (layer "Edge.Cuts"))
 (gr_arc (start 148.86743 132.662376) (mid 148.297624 133.148846) (end 147.689897 133.587022) (stroke (width 0.1) (type default))
  (layer "Edge.Cuts"))
 (gr_line (start 69.640089 90.571905) (end 68.458752 91.129552) (stroke (width 0.1) (type default)) (layer "Edge.Cuts"))
 (gr_line (start 151.017827 78.707882) (end 150.085 77.914306) (stroke (width 0.1) (type default)) (layer "Edge.Cuts"))
 (gr_line (start 82.770366 84.591199) (end 81.630929 85.118519) (stroke (width 0.1) (type default)) (layer "Edge.Cuts"))
 (gr_line (start 58.44206 101.383178) (end 58.231396 101.97091) (stroke (width 0.1) (type default)) (layer "Edge.Cuts"))
 (gr_line (start 129.650573 68.346834) (end 126.679494 68.178844) (stroke (width 0.1) (type default)) (layer "Edge.Cuts"))
 (gr_arc (start 135.129692 138.123718) (mid 134.152338 138.345056) (end 133.165 138.516445) (stroke (width 0.1) (type default))
  (layer "Edge.Cuts"))
 (gr_line (start 79.50006 86.144793) (end 78.231386 86.723764) (stroke (width 0.1) (type default)) (layer "Edge.Cuts"))
 (gr_line (start 154.246525 81.949553) (end 152.935548 80.565403) (stroke (width 0.1) (type default)) (layer "Edge.Cuts"))
 (gr_line (start 160.821561 96.031557) (end 160.319688 93.811023) (stroke (width 0.1) (type default)) (layer "Edge.Cuts"))
 (gr_line (start 68.11456 127.73802) (end 69.265 128.077605) (stroke (width 0.1) (type default)) (layer "Edge.Cuts"))
 (gr_line (start 84.086126 126.34863) (end 85.72089 126.340556) (stroke (width 0.1) (type default)) (layer "Edge.Cuts"))
 (gr_line (start 144.548489 73.266577) (end 142.827845 72.336204) (stroke (width 0.1) (type default)) (layer "Edge.Cuts"))
 (gr_line (start 92.101313 80.109972) (end 91.045 80.772289) (stroke (width 0.1) (type default)) (layer "Edge.Cuts"))
 (gr_line (start 59.494828 98.52696) (end 59.010331 99.777923) (stroke (width 0.1) (type default)) (layer "Edge.Cuts"))
 (gr_arc (start 60.307382 122.487282) (mid 59.699681 121.701005) (end 59.131701 120.885573) (stroke (width 0.1) (type default))
  (layer "Edge.Cuts"))
 (gr_line (start 154.588879 125.842733) (end 155.048661 125.191557) (stroke (width 0.1) (type default)) (layer "Edge.Cuts"))
 (gr_line (start 136.052576 69.533809) (end 134.725 69.166625) (stroke (width 0.1) (type default)) (layer "Edge.Cuts"))
 (gr_line (start 152.935548 80.565403) (end 151.918679 79.544394) (stroke (width 0.1) (type default)) (layer "Edge.Cuts"))
 (gr_line (start 65.983571 126.814619) (end 67.066247 127.336251) (stroke (width 0.1) (type default)) (layer "Edge.Cuts"))
 (gr_line (start 104.879605 133.314834) (end 105.298299 133.532509) (stroke (width 0.1) (type default)) (layer "Edge.Cuts"))
 (segment (start 59.472522 116.782522) (end 59.472522 101.202478) (width 0.2) (layer "F.Cu") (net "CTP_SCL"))
 (segment (start 60.455 117.765) (end 59.472522 116.782522) (width 0.2) (layer "F.Cu") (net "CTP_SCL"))
 (segment (start 62.2 98.475) (end 148.79 98.475) (width 0.2) (layer "F.Cu") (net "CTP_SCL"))
 (segment (start 148.79 98.475) (end 150.925 96.34) (width 0.2) (layer "F.Cu") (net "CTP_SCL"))
 (segment (start 59.472522 101.202478) (end 62.2 98.475) (width 0.2) (layer "F.Cu") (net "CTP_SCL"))
 (segment (start 64.375 121.475) (end 62.975 120.075) (width 0.2) (layer "F.Cu") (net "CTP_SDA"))
 (segment (start 152.36 91.26) (end 152.975 91.875) (width 0.2) (layer "F.Cu") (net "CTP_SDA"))
 (segment (start 154 121.475) (end 64.375 121.475) (width 0.2) (layer "F.Cu") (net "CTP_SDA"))
 (segment (start 152.975 91.875) (end 152.975 120.45) (width 0.2) (layer "F.Cu") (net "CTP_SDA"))
 (segment (start 150.925 91.26) (end 152.36 91.26) (width 0.2) (layer "F.Cu") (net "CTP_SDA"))
 (segment (start 62.995 120.055) (end 62.995 117.765) (width 0.2) (layer "F.Cu") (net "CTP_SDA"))
 (segment (start 62.975 120.075) (end 62.995 120.055) (width 0.2) (layer "F.Cu") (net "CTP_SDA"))
 (segment (start 152.975 120.45) (end 154 121.475) (width 0.2) (layer "F.Cu") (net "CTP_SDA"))
 (segment (start 150.44824 97.491) (end 151.40176 97.491) (width 0.2) (layer "F.Cu") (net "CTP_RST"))
 (segment (start 70.33807 98.876) (end 149.06324 98.876) (width 0.2) (layer "F.Cu") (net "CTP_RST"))
 (segment (start 149.06324 98.876) (end 150.44824 97.491) (width 0.2) (layer "F.Cu") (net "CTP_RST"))
 (segment (start 67.095 116.205) (end 67.095 102.11907) (width 0.2) (layer "F.Cu") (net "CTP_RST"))
 (segment (start 152.076 96.81676) (end 152.076 94.951) (width 0.2) (layer "F.Cu") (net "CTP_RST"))
 (segment (start 67.095 102.11907) (end 70.33807 98.876) (width 0.2) (layer "F.Cu") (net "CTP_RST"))
 (segment (start 151.40176 97.491) (end 152.076 96.81676) (width 0.2) (layer "F.Cu") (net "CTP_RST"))
 (segment (start 152.076 94.951) (end 150.925 93.8) (width 0.2) (layer "F.Cu") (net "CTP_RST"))
 (segment (start 65.535 117.765) (end 67.095 116.205) (width 0.2) (layer "F.Cu") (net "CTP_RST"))
 (segment (start 152.477 93.48624) (end 151.40176 92.411) (width 0.2) (layer "F.Cu") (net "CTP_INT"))
 (segment (start 151.40176 115.271) (end 152.477 114.19576) (width 0.2) (layer "F.Cu") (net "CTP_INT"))
 (segment (start 152.477 114.19576) (end 152.477 93.48624) (width 0.2) (layer "F.Cu") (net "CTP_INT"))
 (segment (start 146.97424 118.745) (end 150.44824 115.271) (width 0.2) (layer "F.Cu") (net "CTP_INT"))
 (segment (start 149.774 91.73676) (end 149.774 89.871) (width 0.2) (layer "F.Cu") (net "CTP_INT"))
 (segment (start 68.075 117.765) (end 69.055 118.745) (width 0.2) (layer "F.Cu") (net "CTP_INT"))
 (segment (start 149.774 89.871) (end 150.925 88.72) (width 0.2) (layer "F.Cu") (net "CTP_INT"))
 (segment (start 150.44824 92.411) (end 149.774 91.73676) (width 0.2) (layer "F.Cu") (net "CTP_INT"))
 (segment (start 150.44824 115.271) (end 151.40176 115.271) (width 0.2) (layer "F.Cu") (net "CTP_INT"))
 (segment (start 151.40176 92.411) (end 150.44824 92.411) (width 0.2) (layer "F.Cu") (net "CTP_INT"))
 (segment (start 69.055 118.745) (end 146.97424 118.745) (width 0.2) (layer "F.Cu") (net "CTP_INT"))
 (segment (start 150.925 109.04) (end 144.415 115.55) (width 0.2) (layer "F.Cu") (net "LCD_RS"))
 (segment (start 92.125 115.525) (end 72.855 115.525) (width 0.2) (layer "F.Cu") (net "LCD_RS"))
 (segment (start 92.15 115.55) (end 92.125 115.525) (width 0.2) (layer "F.Cu") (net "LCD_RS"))
 (segment (start 144.415 115.55) (end 92.15 115.55) (width 0.2) (layer "F.Cu") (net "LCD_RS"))
 (segment (start 72.855 115.525) (end 70.615 117.765) (width 0.2) (layer "F.Cu") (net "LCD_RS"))
 (segment (start 145.955 116.55) (end 116.525 116.55) (width 0.2) (layer "F.Cu") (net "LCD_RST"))
 (segment (start 74.42 116.5) (end 73.155 117.765) (width 0.2) (layer "F.Cu") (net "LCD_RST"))
 (segment (start 116.475 116.5) (end 74.42 116.5) (width 0.2) (layer "F.Cu") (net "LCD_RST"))
 (segment (start 116.525 116.55) (end 116.475 116.5) (width 0.2) (layer "F.Cu") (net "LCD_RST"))
 (segment (start 150.925 111.58) (end 145.955 116.55) (width 0.2) (layer "F.Cu") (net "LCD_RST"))
 (segment (start 150.925 114.12) (end 147.28 117.765) (width 0.2) (layer "F.Cu") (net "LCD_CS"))
 (segment (start 147.28 117.765) (end 75.695 117.765) (width 0.2) (layer "F.Cu") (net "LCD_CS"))
 (segment (start 152.31876 96.574) (end 157.849 96.574) (width 0.2) (layer "B.Cu") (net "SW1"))
 (segment (start 80.57 97.65) (end 151.24276 97.65) (width 0.2) (layer "B.Cu") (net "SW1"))
 (segment (start 151.24276 97.65) (end 152.31876 96.574) (width 0.2) (layer "B.Cu") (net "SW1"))
 (segment (start 157.849 96.574) (end 159.15 97.875) (width 0.2) (layer "B.Cu") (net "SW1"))
 (segment (start 75.695 102.525) (end 80.57 97.65) (width 0.2) (layer "B.Cu") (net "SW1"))
 (segment (start 159.15 97.875) (end 159.15 104.375) (width 0.2) (layer "B.Cu") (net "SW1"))
 (segment (start 76.48 105.85) (end 73.155 102.525) (width 0.2) (layer "F.Cu") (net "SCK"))
 (segment (start 150.925 103.96) (end 149.035 105.85) (width 0.2) (layer "F.Cu") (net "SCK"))
 (segment (start 149.035 105.85) (end 76.48 105.85) (width 0.2) (layer "F.Cu") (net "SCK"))
 (segment (start 150.925 98.88) (end 149.705 100.1) (width 0.2) (layer "F.Cu") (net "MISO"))
 (segment (start 149.705 100.1) (end 71.5 100.1) (width 0.2) (layer "F.Cu") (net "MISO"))
 (segment (start 71.5 100.1) (end 70.615 100.985) (width 0.2) (layer "F.Cu") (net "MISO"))
 (segment (start 70.615 100.985) (end 70.615 102.525) (width 0.2) (layer "F.Cu") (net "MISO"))
 (segment (start 150.925 106.5) (end 69.5 106.5) (width 0.2) (layer "F.Cu") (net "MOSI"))
 (segment (start 69.5 106.5) (end 68.075 105.075) (width 0.2) (layer "F.Cu") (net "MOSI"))
 (segment (start 68.075 105.075) (end 68.075 102.525) (width 0.2) (layer "F.Cu") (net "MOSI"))
 (segment (start 62.995 102.525) (end 65.245 104.775) (width 0.2) (layer "B.Cu") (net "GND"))
 (segment (start 139.04 104.775) (end 150.925 116.66) (width 0.2) (layer "B.Cu") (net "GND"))
 (segment (start 65.245 104.775) (end 139.04 104.775) (width 0.2) (layer "B.Cu") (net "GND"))
 (segment (start 137.075 105.35) (end 150.925 119.2) (width 0.2) (layer "B.Cu") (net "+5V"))
 (segment (start 150.925 119.2) (end 154.25 119.2) (width 0.2) (layer "B.Cu") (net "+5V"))
 (segment (start 154.25 119.2) (end 154.65 118.8) (width 0.2) (layer "B.Cu") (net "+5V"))
 (segment (start 153.88 104.375) (end 154.65 104.375) (width 0.2) (layer "B.Cu") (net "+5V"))
 (segment (start 154.65 97.875) (end 151.105 101.42) (width 0.2) (layer "B.Cu") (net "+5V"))
 (segment (start 150.925 101.42) (end 153.88 104.375) (width 0.2) (layer "B.Cu") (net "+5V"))
 (segment (start 60.455 104.055) (end 61.75 105.35) (width 0.2) (layer "B.Cu") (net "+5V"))
 (segment (start 60.455 102.525) (end 60.455 104.055) (width 0.2) (layer "B.Cu") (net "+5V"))
 (segment (start 61.75 105.35) (end 137.075 105.35) (width 0.2) (layer "B.Cu") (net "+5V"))
 (segment (start 151.105 101.42) (end 150.925 101.42) (width 0.2) (layer "B.Cu") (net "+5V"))
 (segment (start 154.65 118.8) (end 154.65 104.375) (width 0.2) (layer "B.Cu") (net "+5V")))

